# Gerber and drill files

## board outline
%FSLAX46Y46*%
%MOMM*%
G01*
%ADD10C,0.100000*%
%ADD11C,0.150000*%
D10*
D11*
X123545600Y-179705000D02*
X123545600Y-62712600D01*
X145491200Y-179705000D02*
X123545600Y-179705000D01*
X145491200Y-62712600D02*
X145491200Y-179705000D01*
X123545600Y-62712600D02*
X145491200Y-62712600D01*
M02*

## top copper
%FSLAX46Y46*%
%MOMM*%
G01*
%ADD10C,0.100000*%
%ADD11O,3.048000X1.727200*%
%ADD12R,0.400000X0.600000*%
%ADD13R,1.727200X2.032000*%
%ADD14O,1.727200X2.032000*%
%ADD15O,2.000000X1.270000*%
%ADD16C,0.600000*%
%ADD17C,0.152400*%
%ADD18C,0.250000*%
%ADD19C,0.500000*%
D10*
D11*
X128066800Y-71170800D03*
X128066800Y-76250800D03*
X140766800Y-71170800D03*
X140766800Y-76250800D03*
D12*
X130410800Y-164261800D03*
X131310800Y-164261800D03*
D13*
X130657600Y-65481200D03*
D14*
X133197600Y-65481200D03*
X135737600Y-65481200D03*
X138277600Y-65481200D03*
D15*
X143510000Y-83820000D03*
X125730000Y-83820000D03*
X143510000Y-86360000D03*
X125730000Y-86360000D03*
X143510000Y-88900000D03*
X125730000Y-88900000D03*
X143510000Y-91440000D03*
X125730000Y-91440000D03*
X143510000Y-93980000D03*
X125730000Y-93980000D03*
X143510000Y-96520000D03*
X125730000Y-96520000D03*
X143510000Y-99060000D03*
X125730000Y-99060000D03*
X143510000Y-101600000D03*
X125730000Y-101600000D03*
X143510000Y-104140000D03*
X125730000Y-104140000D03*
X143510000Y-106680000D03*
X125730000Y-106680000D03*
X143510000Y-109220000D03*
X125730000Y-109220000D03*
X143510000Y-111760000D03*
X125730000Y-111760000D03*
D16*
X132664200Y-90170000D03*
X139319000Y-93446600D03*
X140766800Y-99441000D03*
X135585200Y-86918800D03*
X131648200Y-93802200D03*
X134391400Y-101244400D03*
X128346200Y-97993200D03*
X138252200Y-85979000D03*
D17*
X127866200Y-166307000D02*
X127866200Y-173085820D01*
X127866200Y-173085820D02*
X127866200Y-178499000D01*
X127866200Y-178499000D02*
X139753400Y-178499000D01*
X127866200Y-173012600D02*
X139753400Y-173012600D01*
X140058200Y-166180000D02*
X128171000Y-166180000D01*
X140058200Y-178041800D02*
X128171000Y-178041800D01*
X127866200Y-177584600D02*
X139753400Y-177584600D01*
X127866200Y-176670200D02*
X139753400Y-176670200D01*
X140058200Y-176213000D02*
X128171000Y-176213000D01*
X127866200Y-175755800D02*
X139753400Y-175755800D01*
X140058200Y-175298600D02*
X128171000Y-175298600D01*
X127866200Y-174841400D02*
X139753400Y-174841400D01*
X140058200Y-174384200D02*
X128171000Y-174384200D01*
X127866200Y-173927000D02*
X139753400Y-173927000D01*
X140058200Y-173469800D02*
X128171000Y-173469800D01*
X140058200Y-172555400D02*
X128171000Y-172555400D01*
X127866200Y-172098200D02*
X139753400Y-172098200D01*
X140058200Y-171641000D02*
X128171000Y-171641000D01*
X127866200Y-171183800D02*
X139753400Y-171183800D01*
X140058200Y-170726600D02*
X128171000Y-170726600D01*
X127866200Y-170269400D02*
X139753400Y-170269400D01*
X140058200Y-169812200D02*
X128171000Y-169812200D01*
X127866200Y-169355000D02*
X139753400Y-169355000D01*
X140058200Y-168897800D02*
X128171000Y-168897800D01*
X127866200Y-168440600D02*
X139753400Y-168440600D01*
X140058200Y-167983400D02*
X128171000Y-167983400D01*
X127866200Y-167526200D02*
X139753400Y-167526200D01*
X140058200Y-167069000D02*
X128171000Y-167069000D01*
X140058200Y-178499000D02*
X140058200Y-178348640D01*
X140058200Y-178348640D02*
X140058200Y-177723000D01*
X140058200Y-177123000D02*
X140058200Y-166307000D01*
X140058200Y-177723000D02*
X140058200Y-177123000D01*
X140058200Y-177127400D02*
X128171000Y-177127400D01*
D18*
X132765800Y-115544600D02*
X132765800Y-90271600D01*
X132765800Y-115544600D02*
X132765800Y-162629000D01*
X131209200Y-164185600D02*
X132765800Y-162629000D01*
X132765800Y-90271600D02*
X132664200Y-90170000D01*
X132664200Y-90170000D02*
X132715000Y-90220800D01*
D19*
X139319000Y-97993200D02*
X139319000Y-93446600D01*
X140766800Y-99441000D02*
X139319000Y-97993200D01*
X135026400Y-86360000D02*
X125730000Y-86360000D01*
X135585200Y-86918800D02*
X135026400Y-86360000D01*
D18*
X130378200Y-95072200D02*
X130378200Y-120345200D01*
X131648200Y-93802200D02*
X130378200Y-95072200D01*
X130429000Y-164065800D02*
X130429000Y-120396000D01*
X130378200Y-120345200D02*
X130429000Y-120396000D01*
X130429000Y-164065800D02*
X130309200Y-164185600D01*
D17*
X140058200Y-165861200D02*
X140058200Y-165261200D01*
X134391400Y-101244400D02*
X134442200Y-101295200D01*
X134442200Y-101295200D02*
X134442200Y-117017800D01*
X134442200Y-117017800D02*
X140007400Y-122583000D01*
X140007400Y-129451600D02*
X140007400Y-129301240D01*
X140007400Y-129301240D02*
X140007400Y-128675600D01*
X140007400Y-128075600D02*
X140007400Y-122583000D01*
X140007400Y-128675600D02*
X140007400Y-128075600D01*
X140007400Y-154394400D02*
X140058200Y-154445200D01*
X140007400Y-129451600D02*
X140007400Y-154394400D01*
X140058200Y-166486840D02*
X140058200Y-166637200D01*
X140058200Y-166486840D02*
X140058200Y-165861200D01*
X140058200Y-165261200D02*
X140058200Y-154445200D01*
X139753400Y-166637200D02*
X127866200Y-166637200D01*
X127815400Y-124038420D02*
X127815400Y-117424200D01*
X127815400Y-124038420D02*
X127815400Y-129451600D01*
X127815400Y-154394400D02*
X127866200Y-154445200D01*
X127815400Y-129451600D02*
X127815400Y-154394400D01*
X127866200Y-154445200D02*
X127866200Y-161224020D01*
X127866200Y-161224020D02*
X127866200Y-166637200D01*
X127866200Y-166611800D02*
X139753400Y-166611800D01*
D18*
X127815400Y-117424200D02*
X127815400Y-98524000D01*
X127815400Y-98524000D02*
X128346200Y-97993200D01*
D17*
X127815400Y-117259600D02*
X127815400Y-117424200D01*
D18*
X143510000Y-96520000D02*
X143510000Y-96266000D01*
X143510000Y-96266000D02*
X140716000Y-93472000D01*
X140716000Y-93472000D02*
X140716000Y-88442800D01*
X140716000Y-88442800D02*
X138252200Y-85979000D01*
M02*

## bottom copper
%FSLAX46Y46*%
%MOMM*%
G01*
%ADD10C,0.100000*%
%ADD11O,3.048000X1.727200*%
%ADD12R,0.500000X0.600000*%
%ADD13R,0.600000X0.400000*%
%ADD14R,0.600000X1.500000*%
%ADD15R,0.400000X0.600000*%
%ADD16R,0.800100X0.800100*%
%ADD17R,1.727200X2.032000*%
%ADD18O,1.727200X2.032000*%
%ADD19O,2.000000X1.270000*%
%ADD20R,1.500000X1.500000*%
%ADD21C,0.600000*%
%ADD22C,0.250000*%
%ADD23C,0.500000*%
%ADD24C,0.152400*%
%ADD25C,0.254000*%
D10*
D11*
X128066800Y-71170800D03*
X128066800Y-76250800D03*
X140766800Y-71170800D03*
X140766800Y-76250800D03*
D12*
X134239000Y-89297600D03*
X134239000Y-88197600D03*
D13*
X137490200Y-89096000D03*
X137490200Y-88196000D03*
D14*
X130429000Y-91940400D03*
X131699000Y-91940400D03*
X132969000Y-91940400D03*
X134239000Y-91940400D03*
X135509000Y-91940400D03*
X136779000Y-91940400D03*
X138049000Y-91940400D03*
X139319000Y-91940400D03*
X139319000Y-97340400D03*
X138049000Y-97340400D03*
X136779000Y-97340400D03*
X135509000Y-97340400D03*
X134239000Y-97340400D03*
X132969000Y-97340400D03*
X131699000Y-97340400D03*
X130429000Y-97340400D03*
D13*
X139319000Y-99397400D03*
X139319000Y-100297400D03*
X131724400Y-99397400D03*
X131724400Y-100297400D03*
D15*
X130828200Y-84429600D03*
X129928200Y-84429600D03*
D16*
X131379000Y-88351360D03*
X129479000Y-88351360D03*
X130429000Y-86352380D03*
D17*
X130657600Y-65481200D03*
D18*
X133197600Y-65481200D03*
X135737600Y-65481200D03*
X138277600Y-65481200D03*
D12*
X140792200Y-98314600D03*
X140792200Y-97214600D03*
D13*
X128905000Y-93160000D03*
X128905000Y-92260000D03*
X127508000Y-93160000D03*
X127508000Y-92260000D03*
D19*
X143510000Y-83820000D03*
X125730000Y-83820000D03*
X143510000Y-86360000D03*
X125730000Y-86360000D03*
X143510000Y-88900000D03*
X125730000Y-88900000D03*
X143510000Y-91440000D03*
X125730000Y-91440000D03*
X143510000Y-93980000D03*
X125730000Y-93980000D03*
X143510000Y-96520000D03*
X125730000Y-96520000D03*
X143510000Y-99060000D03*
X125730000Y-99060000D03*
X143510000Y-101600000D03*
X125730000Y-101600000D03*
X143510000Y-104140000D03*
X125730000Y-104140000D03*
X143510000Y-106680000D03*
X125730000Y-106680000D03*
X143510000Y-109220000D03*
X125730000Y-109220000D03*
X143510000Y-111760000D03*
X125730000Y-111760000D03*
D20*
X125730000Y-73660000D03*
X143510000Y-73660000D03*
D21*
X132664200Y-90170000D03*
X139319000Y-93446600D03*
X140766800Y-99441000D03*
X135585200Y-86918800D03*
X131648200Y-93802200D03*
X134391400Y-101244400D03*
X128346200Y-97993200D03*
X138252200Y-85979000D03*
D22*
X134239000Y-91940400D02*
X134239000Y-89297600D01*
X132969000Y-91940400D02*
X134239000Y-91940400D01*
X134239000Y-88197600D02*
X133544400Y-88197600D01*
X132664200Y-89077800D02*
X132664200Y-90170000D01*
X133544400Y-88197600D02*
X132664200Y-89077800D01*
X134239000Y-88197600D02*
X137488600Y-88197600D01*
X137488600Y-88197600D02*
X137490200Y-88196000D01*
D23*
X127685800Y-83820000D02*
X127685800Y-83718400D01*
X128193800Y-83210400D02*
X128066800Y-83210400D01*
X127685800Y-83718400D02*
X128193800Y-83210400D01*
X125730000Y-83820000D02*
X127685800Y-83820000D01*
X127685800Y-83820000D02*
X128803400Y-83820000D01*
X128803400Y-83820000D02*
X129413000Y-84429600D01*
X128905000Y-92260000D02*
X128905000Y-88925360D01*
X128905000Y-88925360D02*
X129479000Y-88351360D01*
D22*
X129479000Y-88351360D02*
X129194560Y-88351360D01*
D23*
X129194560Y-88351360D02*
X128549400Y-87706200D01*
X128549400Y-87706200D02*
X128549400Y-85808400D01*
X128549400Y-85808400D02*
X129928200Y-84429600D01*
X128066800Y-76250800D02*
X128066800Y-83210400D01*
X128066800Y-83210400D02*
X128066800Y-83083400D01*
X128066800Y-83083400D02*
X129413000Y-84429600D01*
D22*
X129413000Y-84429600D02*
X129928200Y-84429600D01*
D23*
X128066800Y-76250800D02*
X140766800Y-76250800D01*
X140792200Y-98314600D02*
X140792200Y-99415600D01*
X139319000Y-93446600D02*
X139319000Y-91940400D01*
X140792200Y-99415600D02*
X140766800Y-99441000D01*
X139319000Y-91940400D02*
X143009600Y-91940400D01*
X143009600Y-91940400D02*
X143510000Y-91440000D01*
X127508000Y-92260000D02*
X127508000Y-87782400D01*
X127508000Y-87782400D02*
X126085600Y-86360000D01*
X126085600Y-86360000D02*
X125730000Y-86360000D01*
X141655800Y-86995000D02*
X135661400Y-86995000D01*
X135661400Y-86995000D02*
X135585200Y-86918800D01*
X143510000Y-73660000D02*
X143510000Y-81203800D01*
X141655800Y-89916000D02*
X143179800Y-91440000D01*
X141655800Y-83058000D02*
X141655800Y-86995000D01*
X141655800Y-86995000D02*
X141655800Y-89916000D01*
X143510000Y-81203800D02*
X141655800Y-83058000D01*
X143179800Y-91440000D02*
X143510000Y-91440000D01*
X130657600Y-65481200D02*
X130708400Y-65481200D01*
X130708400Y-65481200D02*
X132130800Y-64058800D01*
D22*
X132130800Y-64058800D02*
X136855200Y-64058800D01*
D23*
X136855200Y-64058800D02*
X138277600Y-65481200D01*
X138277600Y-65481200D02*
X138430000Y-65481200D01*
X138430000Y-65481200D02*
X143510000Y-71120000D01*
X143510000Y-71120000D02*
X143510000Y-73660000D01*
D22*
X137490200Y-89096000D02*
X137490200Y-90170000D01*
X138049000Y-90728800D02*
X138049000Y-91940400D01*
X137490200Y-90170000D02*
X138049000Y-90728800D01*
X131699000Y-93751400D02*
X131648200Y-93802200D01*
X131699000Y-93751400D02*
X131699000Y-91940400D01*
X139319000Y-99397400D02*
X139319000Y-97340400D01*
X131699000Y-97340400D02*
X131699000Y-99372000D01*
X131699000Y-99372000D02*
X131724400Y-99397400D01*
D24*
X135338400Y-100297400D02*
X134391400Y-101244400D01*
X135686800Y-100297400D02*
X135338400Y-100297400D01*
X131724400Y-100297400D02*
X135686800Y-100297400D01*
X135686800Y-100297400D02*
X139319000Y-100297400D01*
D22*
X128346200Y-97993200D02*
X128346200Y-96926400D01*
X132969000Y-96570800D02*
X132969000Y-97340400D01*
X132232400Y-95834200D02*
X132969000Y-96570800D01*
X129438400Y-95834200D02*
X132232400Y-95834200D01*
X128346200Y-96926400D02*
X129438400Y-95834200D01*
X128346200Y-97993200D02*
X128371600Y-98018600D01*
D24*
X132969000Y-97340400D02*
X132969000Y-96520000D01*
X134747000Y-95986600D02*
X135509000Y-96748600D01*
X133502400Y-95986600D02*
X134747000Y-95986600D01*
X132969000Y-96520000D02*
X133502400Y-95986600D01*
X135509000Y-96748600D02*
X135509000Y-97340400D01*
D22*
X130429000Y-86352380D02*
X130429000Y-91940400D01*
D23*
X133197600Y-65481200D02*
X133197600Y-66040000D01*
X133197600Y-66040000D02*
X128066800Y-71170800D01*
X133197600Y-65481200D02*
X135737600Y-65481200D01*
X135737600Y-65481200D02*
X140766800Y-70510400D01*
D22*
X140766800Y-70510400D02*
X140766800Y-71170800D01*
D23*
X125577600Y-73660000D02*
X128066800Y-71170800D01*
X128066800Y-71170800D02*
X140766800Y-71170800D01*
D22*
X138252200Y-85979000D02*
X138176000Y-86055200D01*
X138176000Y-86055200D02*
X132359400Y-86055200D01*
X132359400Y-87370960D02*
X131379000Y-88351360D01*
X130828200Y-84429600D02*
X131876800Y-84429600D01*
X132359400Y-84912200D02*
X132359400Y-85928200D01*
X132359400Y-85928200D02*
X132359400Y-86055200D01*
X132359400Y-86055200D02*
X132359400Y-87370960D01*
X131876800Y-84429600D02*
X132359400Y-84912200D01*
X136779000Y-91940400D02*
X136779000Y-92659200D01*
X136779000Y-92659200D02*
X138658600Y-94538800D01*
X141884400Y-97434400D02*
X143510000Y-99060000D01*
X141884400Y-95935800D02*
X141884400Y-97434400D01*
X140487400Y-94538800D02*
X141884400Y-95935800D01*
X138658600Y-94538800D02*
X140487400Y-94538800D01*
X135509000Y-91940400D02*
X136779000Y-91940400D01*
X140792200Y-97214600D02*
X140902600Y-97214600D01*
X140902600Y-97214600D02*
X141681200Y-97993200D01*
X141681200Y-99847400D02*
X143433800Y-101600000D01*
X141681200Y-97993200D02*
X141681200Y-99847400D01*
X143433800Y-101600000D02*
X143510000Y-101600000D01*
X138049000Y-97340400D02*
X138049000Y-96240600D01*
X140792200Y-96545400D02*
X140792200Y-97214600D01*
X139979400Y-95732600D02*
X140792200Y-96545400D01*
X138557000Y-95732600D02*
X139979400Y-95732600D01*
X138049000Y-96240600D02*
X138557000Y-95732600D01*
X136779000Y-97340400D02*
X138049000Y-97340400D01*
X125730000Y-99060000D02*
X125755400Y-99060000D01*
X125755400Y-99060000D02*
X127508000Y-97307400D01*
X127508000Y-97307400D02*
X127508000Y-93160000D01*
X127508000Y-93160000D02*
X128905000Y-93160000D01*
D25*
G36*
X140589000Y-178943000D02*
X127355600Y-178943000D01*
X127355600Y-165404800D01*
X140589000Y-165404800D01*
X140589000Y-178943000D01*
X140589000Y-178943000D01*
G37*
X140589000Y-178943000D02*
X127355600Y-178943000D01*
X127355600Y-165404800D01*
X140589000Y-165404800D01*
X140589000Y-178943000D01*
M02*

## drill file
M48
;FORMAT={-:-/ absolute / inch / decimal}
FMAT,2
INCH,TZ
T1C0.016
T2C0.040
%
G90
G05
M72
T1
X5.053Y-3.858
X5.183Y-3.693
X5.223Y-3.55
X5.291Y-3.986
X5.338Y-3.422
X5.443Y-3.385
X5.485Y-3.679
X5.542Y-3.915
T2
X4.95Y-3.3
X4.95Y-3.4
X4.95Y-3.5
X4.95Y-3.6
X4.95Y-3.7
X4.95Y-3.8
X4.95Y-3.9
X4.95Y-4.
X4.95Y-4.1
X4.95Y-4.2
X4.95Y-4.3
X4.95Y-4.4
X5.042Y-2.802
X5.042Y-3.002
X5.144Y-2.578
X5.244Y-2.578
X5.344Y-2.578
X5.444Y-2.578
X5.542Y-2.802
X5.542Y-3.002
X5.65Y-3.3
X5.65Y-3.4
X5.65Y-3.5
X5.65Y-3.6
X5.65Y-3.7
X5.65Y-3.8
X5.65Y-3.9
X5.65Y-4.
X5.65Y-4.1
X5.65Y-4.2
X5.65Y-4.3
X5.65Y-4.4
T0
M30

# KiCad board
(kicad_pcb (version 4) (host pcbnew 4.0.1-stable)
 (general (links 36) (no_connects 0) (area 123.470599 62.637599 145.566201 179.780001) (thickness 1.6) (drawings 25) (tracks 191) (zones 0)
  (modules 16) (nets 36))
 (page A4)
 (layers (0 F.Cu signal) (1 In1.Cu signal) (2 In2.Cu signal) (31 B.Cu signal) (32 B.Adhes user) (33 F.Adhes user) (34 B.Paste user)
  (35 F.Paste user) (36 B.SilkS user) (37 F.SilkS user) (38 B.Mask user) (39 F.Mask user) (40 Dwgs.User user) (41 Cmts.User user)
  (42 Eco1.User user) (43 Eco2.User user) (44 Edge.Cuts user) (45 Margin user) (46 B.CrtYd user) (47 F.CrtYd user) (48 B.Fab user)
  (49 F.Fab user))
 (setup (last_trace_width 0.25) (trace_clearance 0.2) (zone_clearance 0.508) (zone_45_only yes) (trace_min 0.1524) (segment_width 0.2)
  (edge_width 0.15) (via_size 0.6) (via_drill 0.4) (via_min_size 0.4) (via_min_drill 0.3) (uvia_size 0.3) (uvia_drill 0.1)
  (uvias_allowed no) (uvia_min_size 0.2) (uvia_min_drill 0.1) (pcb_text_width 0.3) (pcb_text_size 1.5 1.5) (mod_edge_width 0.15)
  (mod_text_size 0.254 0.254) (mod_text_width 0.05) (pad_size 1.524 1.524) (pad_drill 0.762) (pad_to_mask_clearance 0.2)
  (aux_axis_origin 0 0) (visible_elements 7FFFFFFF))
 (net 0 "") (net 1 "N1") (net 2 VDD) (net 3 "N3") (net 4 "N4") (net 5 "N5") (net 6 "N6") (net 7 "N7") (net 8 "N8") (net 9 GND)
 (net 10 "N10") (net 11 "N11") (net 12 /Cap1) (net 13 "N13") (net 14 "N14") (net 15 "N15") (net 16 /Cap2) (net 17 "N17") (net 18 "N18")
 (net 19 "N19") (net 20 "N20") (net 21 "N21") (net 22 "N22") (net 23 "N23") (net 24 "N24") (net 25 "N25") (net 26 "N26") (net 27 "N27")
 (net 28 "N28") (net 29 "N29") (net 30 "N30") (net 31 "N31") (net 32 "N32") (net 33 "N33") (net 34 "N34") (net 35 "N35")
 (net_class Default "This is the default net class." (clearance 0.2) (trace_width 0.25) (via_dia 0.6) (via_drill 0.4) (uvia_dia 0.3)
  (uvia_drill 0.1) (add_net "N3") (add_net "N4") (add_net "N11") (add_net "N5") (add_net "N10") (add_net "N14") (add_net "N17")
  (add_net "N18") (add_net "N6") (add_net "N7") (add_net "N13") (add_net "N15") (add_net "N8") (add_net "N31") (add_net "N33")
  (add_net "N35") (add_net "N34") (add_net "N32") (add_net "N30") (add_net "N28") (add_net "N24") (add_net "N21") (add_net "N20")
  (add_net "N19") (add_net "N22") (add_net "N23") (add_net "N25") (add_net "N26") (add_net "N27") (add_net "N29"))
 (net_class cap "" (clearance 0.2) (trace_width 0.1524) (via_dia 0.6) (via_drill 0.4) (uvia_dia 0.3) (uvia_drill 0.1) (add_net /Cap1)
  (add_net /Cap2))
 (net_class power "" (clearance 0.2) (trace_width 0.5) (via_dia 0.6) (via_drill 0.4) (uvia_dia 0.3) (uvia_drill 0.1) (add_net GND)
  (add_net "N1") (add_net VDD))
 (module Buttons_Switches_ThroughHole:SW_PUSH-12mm (layer B.Cu) (at 134.4168 73.7108 180)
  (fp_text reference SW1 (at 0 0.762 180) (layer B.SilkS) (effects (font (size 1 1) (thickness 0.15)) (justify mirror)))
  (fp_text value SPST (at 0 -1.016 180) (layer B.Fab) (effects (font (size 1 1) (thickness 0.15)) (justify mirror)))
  (pad 1 thru_hole oval (at 6.35 2.54 180) (size 3.048 1.7272) (drill 1.016) (layers *.Cu *.Mask B.SilkS) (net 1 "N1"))
  (pad 2 thru_hole oval (at 6.35 -2.54 180) (size 3.048 1.7272) (drill 1.016) (layers *.Cu *.Mask B.SilkS) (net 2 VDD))
  (pad 1 thru_hole oval (at -6.35 2.54 180) (size 3.048 1.7272) (drill 1.016) (layers *.Cu *.Mask B.SilkS) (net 1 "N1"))
  (pad 2 thru_hole oval (at -6.35 -2.54 180) (size 3.048 1.7272) (drill 1.016) (layers *.Cu *.Mask B.SilkS) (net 2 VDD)))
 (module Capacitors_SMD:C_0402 (layer B.Cu) (at 134.239 88.7476 90)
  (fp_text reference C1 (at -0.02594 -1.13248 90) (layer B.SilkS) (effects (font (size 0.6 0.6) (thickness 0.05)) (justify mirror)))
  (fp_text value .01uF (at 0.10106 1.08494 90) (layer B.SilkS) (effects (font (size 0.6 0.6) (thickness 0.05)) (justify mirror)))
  (pad 1 smd rect (at -0.55 0 90) (size 0.6 0.5) (layers B.Cu B.Paste B.Mask) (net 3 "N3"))
  (pad 2 smd rect (at 0.55 0 90) (size 0.6 0.5) (layers B.Cu B.Paste B.Mask) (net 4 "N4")))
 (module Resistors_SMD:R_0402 (layer B.Cu) (at 137.4902 88.646 90)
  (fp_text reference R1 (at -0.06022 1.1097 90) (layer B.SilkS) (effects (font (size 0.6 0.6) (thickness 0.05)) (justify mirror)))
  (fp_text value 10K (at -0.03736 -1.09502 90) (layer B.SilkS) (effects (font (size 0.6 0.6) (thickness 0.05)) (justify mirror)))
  (pad 1 smd rect (at -0.45 0 90) (size 0.4 0.6) (layers B.Cu B.Paste B.Mask) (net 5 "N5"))
  (pad 2 smd rect (at 0.45 0 90) (size 0.4 0.6) (layers B.Cu B.Paste B.Mask) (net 4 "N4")))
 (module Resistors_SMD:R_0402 (layer F.Cu) (at 130.8608 164.2618)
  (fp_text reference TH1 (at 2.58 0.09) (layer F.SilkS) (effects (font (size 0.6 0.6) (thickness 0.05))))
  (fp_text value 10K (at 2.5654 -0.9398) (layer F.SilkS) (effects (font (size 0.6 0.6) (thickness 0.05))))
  (pad 1 smd rect (at -0.45 0) (size 0.4 0.6) (layers F.Cu F.Paste F.Mask) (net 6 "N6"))
  (pad 2 smd rect (at 0.45 0) (size 0.4 0.6) (layers F.Cu F.Paste F.Mask) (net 4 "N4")))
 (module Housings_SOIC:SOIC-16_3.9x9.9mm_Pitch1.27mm (layer B.Cu) (at 134.874 94.6404 270)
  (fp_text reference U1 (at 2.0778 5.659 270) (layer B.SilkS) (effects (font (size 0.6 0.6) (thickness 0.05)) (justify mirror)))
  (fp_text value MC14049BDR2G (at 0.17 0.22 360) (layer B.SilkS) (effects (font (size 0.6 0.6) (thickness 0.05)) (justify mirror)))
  (pad 1 smd rect (at -2.7 4.445 270) (size 1.5 0.6) (layers B.Cu B.Paste B.Mask) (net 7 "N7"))
  (pad 2 smd rect (at -2.7 3.175 270) (size 1.5 0.6) (layers B.Cu B.Paste B.Mask) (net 6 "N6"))
  (pad 3 smd rect (at -2.7 1.905 270) (size 1.5 0.6) (layers B.Cu B.Paste B.Mask) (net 3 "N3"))
  (pad 4 smd rect (at -2.7 0.635 270) (size 1.5 0.6) (layers B.Cu B.Paste B.Mask) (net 3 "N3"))
  (pad 5 smd rect (at -2.7 -0.635 270) (size 1.5 0.6) (layers B.Cu B.Paste B.Mask) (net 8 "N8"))
  (pad 6 smd rect (at -2.7 -1.905 270) (size 1.5 0.6) (layers B.Cu B.Paste B.Mask) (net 8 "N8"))
  (pad 7 smd rect (at -2.7 -3.175 270) (size 1.5 0.6) (layers B.Cu B.Paste B.Mask) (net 5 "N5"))
  (pad 8 smd rect (at -2.7 -4.445 270) (size 1.5 0.6) (layers B.Cu B.Paste B.Mask) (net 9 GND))
  (pad 9 smd rect (at 2.7 -4.445 270) (size 1.5 0.6) (layers B.Cu B.Paste B.Mask) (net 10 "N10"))
  (pad 10 smd rect (at 2.7 -3.175 270) (size 1.5 0.6) (layers B.Cu B.Paste B.Mask) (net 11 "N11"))
  (pad 11 smd rect (at 2.7 -1.905 270) (size 1.5 0.6) (layers B.Cu B.Paste B.Mask) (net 11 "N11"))
  (pad 12 smd rect (at 2.7 -0.635 270) (size 1.5 0.6) (layers B.Cu B.Paste B.Mask) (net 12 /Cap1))
  (pad 13 smd rect (at 2.7 0.635 270) (size 1.5 0.6) (layers B.Cu B.Paste B.Mask) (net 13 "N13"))
  (pad 14 smd rect (at 2.7 1.905 270) (size 1.5 0.6) (layers B.Cu B.Paste B.Mask) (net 12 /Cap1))
  (pad 15 smd rect (at 2.7 3.175 270) (size 1.5 0.6) (layers B.Cu B.Paste B.Mask) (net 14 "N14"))
  (pad 16 smd rect (at 2.7 4.445 270) (size 1.5 0.6) (layers B.Cu B.Paste B.Mask) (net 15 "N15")))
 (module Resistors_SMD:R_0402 (layer B.Cu) (at 139.319 99.8474 270)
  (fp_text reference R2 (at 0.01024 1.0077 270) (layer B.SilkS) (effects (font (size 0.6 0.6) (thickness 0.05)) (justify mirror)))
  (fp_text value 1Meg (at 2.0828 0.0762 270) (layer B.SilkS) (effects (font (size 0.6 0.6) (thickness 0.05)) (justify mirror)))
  (pad 1 smd rect (at -0.45 0 270) (size 0.4 0.6) (layers B.Cu B.Paste B.Mask) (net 10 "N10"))
  (pad 2 smd rect (at 0.45 0 270) (size 0.4 0.6) (layers B.Cu B.Paste B.Mask) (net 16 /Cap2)))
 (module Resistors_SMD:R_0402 (layer B.Cu) (at 131.7244 99.8474 270)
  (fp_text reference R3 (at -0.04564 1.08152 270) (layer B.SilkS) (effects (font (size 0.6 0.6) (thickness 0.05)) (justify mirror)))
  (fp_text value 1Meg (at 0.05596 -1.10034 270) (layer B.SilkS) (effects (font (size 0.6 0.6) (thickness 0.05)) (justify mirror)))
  (pad 1 smd rect (at -0.45 0 270) (size 0.4 0.6) (layers B.Cu B.Paste B.Mask) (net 14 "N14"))
  (pad 2 smd rect (at 0.45 0 270) (size 0.4 0.6) (layers B.Cu B.Paste B.Mask) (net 16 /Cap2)))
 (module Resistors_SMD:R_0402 (layer B.Cu) (at 130.3782 84.4296 180)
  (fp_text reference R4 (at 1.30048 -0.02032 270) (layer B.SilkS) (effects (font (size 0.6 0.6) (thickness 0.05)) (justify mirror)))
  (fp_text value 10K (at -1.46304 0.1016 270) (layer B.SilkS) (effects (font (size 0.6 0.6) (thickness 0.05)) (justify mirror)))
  (pad 1 smd rect (at -0.45 0 180) (size 0.4 0.6) (layers B.Cu B.Paste B.Mask) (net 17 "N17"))
  (pad 2 smd rect (at 0.45 0 180) (size 0.4 0.6) (layers B.Cu B.Paste B.Mask) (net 2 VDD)))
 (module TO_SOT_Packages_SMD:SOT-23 (layer B.Cu) (at 130.429 87.3506 180)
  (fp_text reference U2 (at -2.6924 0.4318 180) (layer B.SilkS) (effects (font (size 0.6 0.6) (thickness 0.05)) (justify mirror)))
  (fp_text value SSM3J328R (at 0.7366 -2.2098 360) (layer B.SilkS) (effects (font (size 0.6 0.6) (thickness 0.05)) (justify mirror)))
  (pad 1 smd rect (at -0.95 -1.00076 180) (size 0.8001 0.8001) (layers B.Cu B.Paste B.Mask) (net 17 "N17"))
  (pad 2 smd rect (at 0.95 -1.00076 180) (size 0.8001 0.8001) (layers B.Cu B.Paste B.Mask) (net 2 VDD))
  (pad 3 smd rect (at 0 0.99822 180) (size 0.8001 0.8001) (layers B.Cu B.Paste B.Mask) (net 7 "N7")))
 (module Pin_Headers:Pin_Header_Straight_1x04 (layer F.Cu) (at 130.6576 65.4812 90)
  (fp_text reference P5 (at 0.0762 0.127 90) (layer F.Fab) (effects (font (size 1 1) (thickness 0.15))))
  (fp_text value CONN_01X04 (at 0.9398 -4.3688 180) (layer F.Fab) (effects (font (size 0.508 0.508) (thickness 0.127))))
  (pad 1 thru_hole rect (at 0 0 90) (size 2.032 1.7272) (drill 1.016) (layers *.Cu *.Mask F.SilkS) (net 9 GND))
  (pad 2 thru_hole oval (at 0 2.54 90) (size 2.032 1.7272) (drill 1.016) (layers *.Cu *.Mask F.SilkS) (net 1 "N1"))
  (pad 3 thru_hole oval (at 0 5.08 90) (size 2.032 1.7272) (drill 1.016) (layers *.Cu *.Mask F.SilkS) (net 1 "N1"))
  (pad 4 thru_hole oval (at 0 7.62 90) (size 2.032 1.7272) (drill 1.016) (layers *.Cu *.Mask F.SilkS) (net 9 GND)))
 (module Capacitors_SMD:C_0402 (layer B.Cu) (at 140.7922 97.7646 90)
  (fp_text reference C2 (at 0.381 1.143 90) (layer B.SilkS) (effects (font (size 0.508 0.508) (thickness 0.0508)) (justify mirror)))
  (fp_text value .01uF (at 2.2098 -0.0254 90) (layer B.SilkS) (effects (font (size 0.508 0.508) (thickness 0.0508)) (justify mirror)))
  (pad 1 smd rect (at -0.55 0 90) (size 0.6 0.5) (layers B.Cu B.Paste B.Mask) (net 9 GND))
  (pad 2 smd rect (at 0.55 0 90) (size 0.6 0.5) (layers B.Cu B.Paste B.Mask) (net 11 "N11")))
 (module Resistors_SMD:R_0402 (layer B.Cu) (at 128.905 92.71 90)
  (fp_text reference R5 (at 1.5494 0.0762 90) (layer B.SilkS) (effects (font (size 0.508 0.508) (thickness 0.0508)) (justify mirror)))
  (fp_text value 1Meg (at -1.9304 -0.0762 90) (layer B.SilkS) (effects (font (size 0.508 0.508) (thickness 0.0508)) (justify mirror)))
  (pad 1 smd rect (at -0.45 0 90) (size 0.4 0.6) (layers B.Cu B.Paste B.Mask) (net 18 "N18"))
  (pad 2 smd rect (at 0.45 0 90) (size 0.4 0.6) (layers B.Cu B.Paste B.Mask) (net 2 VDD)))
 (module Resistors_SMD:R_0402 (layer B.Cu) (at 127.508 92.71 90)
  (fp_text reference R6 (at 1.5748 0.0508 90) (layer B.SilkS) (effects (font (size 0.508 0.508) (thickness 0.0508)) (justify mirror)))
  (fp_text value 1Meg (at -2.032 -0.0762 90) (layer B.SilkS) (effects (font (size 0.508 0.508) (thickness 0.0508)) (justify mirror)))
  (pad 1 smd rect (at -0.45 0 90) (size 0.4 0.6) (layers B.Cu B.Paste B.Mask) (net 18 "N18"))
  (pad 2 smd rect (at 0.45 0 90) (size 0.4 0.6) (layers B.Cu B.Paste B.Mask) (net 9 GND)))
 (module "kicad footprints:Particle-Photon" (layer F.Cu) (at 134.62 97.79 270)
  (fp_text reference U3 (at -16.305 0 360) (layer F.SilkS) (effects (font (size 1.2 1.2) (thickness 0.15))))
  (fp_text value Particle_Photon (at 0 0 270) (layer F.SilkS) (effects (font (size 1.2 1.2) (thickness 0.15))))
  (pad 24 thru_hole oval (at -13.97 -8.89 270) (size 1.27 2) (drill 1.016) (layers *.Cu *.Mask F.SilkS) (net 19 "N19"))
  (pad 1 thru_hole oval (at -13.97 8.89 270) (size 1.27 2) (drill 1.016) (layers *.Cu *.Mask F.SilkS) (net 2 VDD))
  (pad 23 thru_hole oval (at -11.43 -8.89 270) (size 1.27 2) (drill 1.016) (layers *.Cu *.Mask F.SilkS) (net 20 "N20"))
  (pad 2 thru_hole oval (at -11.43 8.89 270) (size 1.27 2) (drill 1.016) (layers *.Cu *.Mask F.SilkS) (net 9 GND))
  (pad 22 thru_hole oval (at -8.89 -8.89 270) (size 1.27 2) (drill 1.016) (layers *.Cu *.Mask F.SilkS) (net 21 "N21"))
  (pad 3 thru_hole oval (at -8.89 8.89 270) (size 1.27 2) (drill 1.016) (layers *.Cu *.Mask F.SilkS) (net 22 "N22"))
  (pad 21 thru_hole oval (at -6.35 -8.89 270) (size 1.27 2) (drill 1.016) (layers *.Cu *.Mask F.SilkS) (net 9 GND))
  (pad 4 thru_hole oval (at -6.35 8.89 270) (size 1.27 2) (drill 1.016) (layers *.Cu *.Mask F.SilkS) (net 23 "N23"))
  (pad 20 thru_hole oval (at -3.81 -8.89 270) (size 1.27 2) (drill 1.016) (layers *.Cu *.Mask F.SilkS) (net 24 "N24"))
  (pad 5 thru_hole oval (at -3.81 8.89 270) (size 1.27 2) (drill 1.016) (layers *.Cu *.Mask F.SilkS) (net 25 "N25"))
  (pad 19 thru_hole oval (at -1.27 -8.89 270) (size 1.27 2) (drill 1.016) (layers *.Cu *.Mask F.SilkS) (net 17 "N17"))
  (pad 6 thru_hole oval (at -1.27 8.89 270) (size 1.27 2) (drill 1.016) (layers *.Cu *.Mask F.SilkS) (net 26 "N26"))
  (pad 18 thru_hole oval (at 1.27 -8.89 270) (size 1.27 2) (drill 1.016) (layers *.Cu *.Mask F.SilkS) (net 8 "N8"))
  (pad 7 thru_hole oval (at 1.27 8.89 270) (size 1.27 2) (drill 1.016) (layers *.Cu *.Mask F.SilkS) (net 18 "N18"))
  (pad 17 thru_hole oval (at 3.81 -8.89 270) (size 1.27 2) (drill 1.016) (layers *.Cu *.Mask F.SilkS) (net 11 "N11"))
  (pad 8 thru_hole oval (at 3.81 8.89 270) (size 1.27 2) (drill 1.016) (layers *.Cu *.Mask F.SilkS) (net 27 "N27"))
  (pad 16 thru_hole oval (at 6.35 -8.89 270) (size 1.27 2) (drill 1.016) (layers *.Cu *.Mask F.SilkS) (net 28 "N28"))
  (pad 9 thru_hole oval (at 6.35 8.89 270) (size 1.27 2) (drill 1.016) (layers *.Cu *.Mask F.SilkS) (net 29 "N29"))
  (pad 15 thru_hole oval (at 8.89 -8.89 270) (size 1.27 2) (drill 1.016) (layers *.Cu *.Mask F.SilkS) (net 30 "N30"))
  (pad 10 thru_hole oval (at 8.89 8.89 270) (size 1.27 2) (drill 1.016) (layers *.Cu *.Mask F.SilkS) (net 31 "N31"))
  (pad 14 thru_hole oval (at 11.43 -8.89 270) (size 1.27 2) (drill 1.016) (layers *.Cu *.Mask F.SilkS) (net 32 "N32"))
  (pad 11 thru_hole oval (at 11.43 8.89 270) (size 1.27 2) (drill 1.016) (layers *.Cu *.Mask F.SilkS) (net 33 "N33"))
  (pad 13 thru_hole oval (at 13.97 -8.89 270) (size 1.27 2) (drill 1.016) (layers *.Cu *.Mask F.SilkS) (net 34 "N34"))
  (pad 12 thru_hole oval (at 13.97 8.89 270) (size 1.27 2) (drill 1.016) (layers *.Cu *.Mask F.SilkS) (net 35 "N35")))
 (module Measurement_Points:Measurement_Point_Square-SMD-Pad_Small (layer B.Cu) (at 125.73 73.66)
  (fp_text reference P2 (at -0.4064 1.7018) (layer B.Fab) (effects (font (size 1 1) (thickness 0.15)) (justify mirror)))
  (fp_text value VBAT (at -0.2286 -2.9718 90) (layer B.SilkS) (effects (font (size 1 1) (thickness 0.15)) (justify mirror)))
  (pad 1 smd rect (at 0 0) (size 1.5 1.5) (layers B.Cu B.Mask) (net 1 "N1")))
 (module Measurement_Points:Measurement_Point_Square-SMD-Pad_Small (layer B.Cu) (at 143.51 73.66)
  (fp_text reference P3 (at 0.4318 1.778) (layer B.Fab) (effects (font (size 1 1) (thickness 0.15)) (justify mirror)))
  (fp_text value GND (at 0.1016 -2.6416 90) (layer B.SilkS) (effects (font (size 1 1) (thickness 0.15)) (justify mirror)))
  (pad 1 smd rect (at 0 0) (size 1.5 1.5) (layers B.Cu B.Mask) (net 9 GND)))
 (gr_line (start 123.5456 179.705) (end 123.5456 62.7126) (angle 90) (layer Edge.Cuts) (width 0.15))
 (gr_line (start 145.4912 179.705) (end 123.5456 179.705) (angle 90) (layer Edge.Cuts) (width 0.15))
 (gr_line (start 145.4912 62.7126) (end 145.4912 179.705) (angle 90) (layer Edge.Cuts) (width 0.15))
 (gr_line (start 123.5456 62.7126) (end 145.4912 62.7126) (angle 90) (layer Edge.Cuts) (width 0.15))
 (segment (start 127.8662 166.307) (end 127.8662 173.08582) (width 0.1524) (layer F.Cu) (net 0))
 (segment (start 127.8662 173.08582) (end 127.8662 178.499) (width 0.1524) (layer F.Cu) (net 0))
 (segment (start 127.8662 178.499) (end 139.7534 178.499) (width 0.1524) (layer F.Cu) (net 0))
 (segment (start 127.8662 173.0126) (end 139.7534 173.0126) (width 0.1524) (layer F.Cu) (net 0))
 (segment (start 140.0582 166.18) (end 128.171 166.18) (width 0.1524) (layer F.Cu) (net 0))
 (segment (start 140.0582 178.0418) (end 128.171 178.0418) (width 0.1524) (layer F.Cu) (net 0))
 (segment (start 127.8662 177.5846) (end 139.7534 177.5846) (width 0.1524) (layer F.Cu) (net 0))
 (segment (start 127.8662 176.6702) (end 139.7534 176.6702) (width 0.1524) (layer F.Cu) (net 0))
 (segment (start 140.0582 176.213) (end 128.171 176.213) (width 0.1524) (layer F.Cu) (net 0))
 (segment (start 127.8662 175.7558) (end 139.7534 175.7558) (width 0.1524) (layer F.Cu) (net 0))
 (segment (start 140.0582 175.2986) (end 128.171 175.2986) (width 0.1524) (layer F.Cu) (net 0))
 (segment (start 127.8662 174.8414) (end 139.7534 174.8414) (width 0.1524) (layer F.Cu) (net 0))
 (segment (start 140.0582 174.3842) (end 128.171 174.3842) (width 0.1524) (layer F.Cu) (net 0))
 (segment (start 127.8662 173.927) (end 139.7534 173.927) (width 0.1524) (layer F.Cu) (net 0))
 (segment (start 140.0582 173.4698) (end 128.171 173.4698) (width 0.1524) (layer F.Cu) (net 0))
 (segment (start 140.0582 172.5554) (end 128.171 172.5554) (width 0.1524) (layer F.Cu) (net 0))
 (segment (start 127.8662 172.0982) (end 139.7534 172.0982) (width 0.1524) (layer F.Cu) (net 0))
 (segment (start 140.0582 171.641) (end 128.171 171.641) (width 0.1524) (layer F.Cu) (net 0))
 (segment (start 127.8662 171.1838) (end 139.7534 171.1838) (width 0.1524) (layer F.Cu) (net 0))
 (segment (start 140.0582 170.7266) (end 128.171 170.7266) (width 0.1524) (layer F.Cu) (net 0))
 (segment (start 127.8662 170.2694) (end 139.7534 170.2694) (width 0.1524) (layer F.Cu) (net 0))
 (segment (start 140.0582 169.8122) (end 128.171 169.8122) (width 0.1524) (layer F.Cu) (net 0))
 (segment (start 127.8662 169.355) (end 139.7534 169.355) (width 0.1524) (layer F.Cu) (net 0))
 (segment (start 140.0582 168.8978) (end 128.171 168.8978) (width 0.1524) (layer F.Cu) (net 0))
 (segment (start 127.8662 168.4406) (end 139.7534 168.4406) (width 0.1524) (layer F.Cu) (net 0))
 (segment (start 140.0582 167.9834) (end 128.171 167.9834) (width 0.1524) (layer F.Cu) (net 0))
 (segment (start 127.8662 167.5262) (end 139.7534 167.5262) (width 0.1524) (layer F.Cu) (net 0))
 (segment (start 140.0582 167.069) (end 128.171 167.069) (width 0.1524) (layer F.Cu) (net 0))
 (segment (start 140.0582 178.499) (end 140.0582 178.34864) (width 0.1524) (layer F.Cu) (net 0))
 (segment (start 140.0582 178.34864) (end 140.0582 177.723) (width 0.1524) (layer F.Cu) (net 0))
 (segment (start 140.0582 177.123) (end 140.0582 166.307) (width 0.1524) (layer F.Cu) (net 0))
 (segment (start 140.0582 177.723) (end 140.0582 177.123) (width 0.1524) (layer F.Cu) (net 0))
 (segment (start 140.0582 177.1274) (end 128.171 177.1274) (width 0.1524) (layer F.Cu) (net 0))
 (segment (start 134.239 91.9404) (end 134.239 89.2976) (width 0.25) (layer B.Cu) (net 3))
 (segment (start 132.969 91.9404) (end 134.239 91.9404) (width 0.25) (layer B.Cu) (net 3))
 (segment (start 132.7658 115.5446) (end 132.7658 90.2716) (width 0.25) (layer F.Cu) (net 4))
 (segment (start 132.7658 115.5446) (end 132.7658 162.629) (width 0.25) (layer F.Cu) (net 4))
 (segment (start 131.2092 164.1856) (end 132.7658 162.629) (width 0.25) (layer F.Cu) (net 4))
 (segment (start 132.7658 90.2716) (end 132.6642 90.17) (width 0.25) (layer F.Cu) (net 4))
 (segment (start 134.239 88.1976) (end 133.5444 88.1976) (width 0.25) (layer B.Cu) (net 4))
 (segment (start 132.6642 90.17) (end 132.715 90.2208) (width 0.25) (layer F.Cu) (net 4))
 (via (at 132.6642 90.17) (size 0.6) (drill 0.4) (layers F.Cu B.Cu) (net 4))
 (segment (start 132.6642 89.0778) (end 132.6642 90.17) (width 0.25) (layer B.Cu) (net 4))
 (segment (start 133.5444 88.1976) (end 132.6642 89.0778) (width 0.25) (layer B.Cu) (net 4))
 (segment (start 134.239 88.1976) (end 137.4886 88.1976) (width 0.25) (layer B.Cu) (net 4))
 (segment (start 137.4886 88.1976) (end 137.4902 88.196) (width 0.25) (layer B.Cu) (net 4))
 (segment (start 127.6858 83.82) (end 127.6858 83.7184) (width 0.5) (layer B.Cu) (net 2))
 (segment (start 128.1938 83.2104) (end 128.0668 83.2104) (width 0.5) (layer B.Cu) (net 2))
 (segment (start 127.6858 83.7184) (end 128.1938 83.2104) (width 0.5) (layer B.Cu) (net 2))
 (segment (start 125.73 83.82) (end 127.6858 83.82) (width 0.5) (layer B.Cu) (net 2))
 (segment (start 127.6858 83.82) (end 128.8034 83.82) (width 0.5) (layer B.Cu) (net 2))
 (segment (start 128.8034 83.82) (end 129.413 84.4296) (width 0.5) (layer B.Cu) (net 2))
 (segment (start 128.905 92.26) (end 128.905 88.92536) (width 0.5) (layer B.Cu) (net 2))
 (segment (start 128.905 88.92536) (end 129.479 88.35136) (width 0.5) (layer B.Cu) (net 2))
 (segment (start 129.479 88.35136) (end 129.19456 88.35136) (width 0.25) (layer B.Cu) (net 2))
 (segment (start 129.19456 88.35136) (end 128.5494 87.7062) (width 0.5) (layer B.Cu) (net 2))
 (segment (start 128.5494 87.7062) (end 128.5494 85.8084) (width 0.5) (layer B.Cu) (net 2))
 (segment (start 128.5494 85.8084) (end 129.9282 84.4296) (width 0.5) (layer B.Cu) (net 2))
 (segment (start 128.0668 76.2508) (end 128.0668 83.2104) (width 0.5) (layer B.Cu) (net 2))
 (segment (start 128.0668 83.2104) (end 128.0668 83.0834) (width 0.5) (layer B.Cu) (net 2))
 (segment (start 128.0668 83.0834) (end 129.413 84.4296) (width 0.5) (layer B.Cu) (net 2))
 (segment (start 129.413 84.4296) (end 129.9282 84.4296) (width 0.25) (layer B.Cu) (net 2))
 (segment (start 128.0668 76.2508) (end 140.7668 76.2508) (width 0.5) (layer B.Cu) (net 2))
 (segment (start 140.7922 98.3146) (end 140.7922 99.4156) (width 0.5) (layer B.Cu) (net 9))
 (segment (start 139.319 93.4466) (end 139.319 91.9404) (width 0.5) (layer B.Cu) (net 9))
 (via (at 139.319 93.4466) (size 0.6) (drill 0.4) (layers F.Cu B.Cu) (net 9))
 (segment (start 139.319 97.9932) (end 139.319 93.4466) (width 0.5) (layer F.Cu) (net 9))
 (segment (start 140.7668 99.441) (end 139.319 97.9932) (width 0.5) (layer F.Cu) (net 9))
 (via (at 140.7668 99.441) (size 0.6) (drill 0.4) (layers F.Cu B.Cu) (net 9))
 (segment (start 140.7922 99.4156) (end 140.7668 99.441) (width 0.5) (layer B.Cu) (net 9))
 (segment (start 139.319 91.9404) (end 143.0096 91.9404) (width 0.5) (layer B.Cu) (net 9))
 (segment (start 143.0096 91.9404) (end 143.51 91.44) (width 0.5) (layer B.Cu) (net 9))
 (segment (start 127.508 92.26) (end 127.508 87.7824) (width 0.5) (layer B.Cu) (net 9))
 (segment (start 127.508 87.7824) (end 126.0856 86.36) (width 0.5) (layer B.Cu) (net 9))
 (segment (start 126.0856 86.36) (end 125.73 86.36) (width 0.5) (layer B.Cu) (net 9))
 (segment (start 141.6558 86.995) (end 135.6614 86.995) (width 0.5) (layer B.Cu) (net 9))
 (segment (start 135.0264 86.36) (end 125.73 86.36) (width 0.5) (layer F.Cu) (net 9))
 (segment (start 135.5852 86.9188) (end 135.0264 86.36) (width 0.5) (layer F.Cu) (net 9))
 (via (at 135.5852 86.9188) (size 0.6) (drill 0.4) (layers F.Cu B.Cu) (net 9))
 (segment (start 135.6614 86.995) (end 135.5852 86.9188) (width 0.5) (layer B.Cu) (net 9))
 (segment (start 143.51 73.66) (end 143.51 81.2038) (width 0.5) (layer B.Cu) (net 9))
 (segment (start 141.6558 89.916) (end 143.1798 91.44) (width 0.5) (layer B.Cu) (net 9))
 (segment (start 141.6558 83.058) (end 141.6558 86.995) (width 0.5) (layer B.Cu) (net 9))
 (segment (start 141.6558 86.995) (end 141.6558 89.916) (width 0.5) (layer B.Cu) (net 9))
 (segment (start 143.51 81.2038) (end 141.6558 83.058) (width 0.5) (layer B.Cu) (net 9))
 (segment (start 143.1798 91.44) (end 143.51 91.44) (width 0.5) (layer B.Cu) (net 9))
 (segment (start 130.6576 65.4812) (end 130.7084 65.4812) (width 0.5) (layer B.Cu) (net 9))
 (segment (start 130.7084 65.4812) (end 132.1308 64.0588) (width 0.5) (layer B.Cu) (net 9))
 (segment (start 132.1308 64.0588) (end 136.8552 64.0588) (width 0.25) (layer B.Cu) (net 9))
 (segment (start 136.8552 64.0588) (end 138.2776 65.4812) (width 0.5) (layer B.Cu) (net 9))
 (segment (start 138.2776 65.4812) (end 138.43 65.4812) (width 0.5) (layer B.Cu) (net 9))
 (segment (start 138.43 65.4812) (end 143.51 71.12) (width 0.5) (layer B.Cu) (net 9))
 (segment (start 143.51 71.12) (end 143.51 73.66) (width 0.5) (layer B.Cu) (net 9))
 (segment (start 137.4902 89.096) (end 137.4902 90.17) (width 0.25) (layer B.Cu) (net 5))
 (segment (start 138.049 90.7288) (end 138.049 91.9404) (width 0.25) (layer B.Cu) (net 5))
 (segment (start 137.4902 90.17) (end 138.049 90.7288) (width 0.25) (layer B.Cu) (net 5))
 (segment (start 130.3782 95.0722) (end 130.3782 120.3452) (width 0.25) (layer F.Cu) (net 6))
 (segment (start 131.699 93.7514) (end 131.6482 93.8022) (width 0.25) (layer B.Cu) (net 6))
 (via (at 131.6482 93.8022) (size 0.6) (drill 0.4) (layers F.Cu B.Cu) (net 6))
 (segment (start 131.6482 93.8022) (end 130.3782 95.0722) (width 0.25) (layer F.Cu) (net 6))
 (segment (start 130.429 164.0658) (end 130.429 120.396) (width 0.25) (layer F.Cu) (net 6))
 (segment (start 131.699 93.7514) (end 131.699 91.9404) (width 0.25) (layer B.Cu) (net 6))
 (segment (start 130.3782 120.3452) (end 130.429 120.396) (width 0.25) (layer F.Cu) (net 6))
 (segment (start 130.429 164.0658) (end 130.3092 164.1856) (width 0.25) (layer F.Cu) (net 6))
 (segment (start 139.319 99.3974) (end 139.319 97.3404) (width 0.25) (layer B.Cu) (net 10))
 (segment (start 131.699 97.3404) (end 131.699 99.372) (width 0.25) (layer B.Cu) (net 14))
 (segment (start 131.699 99.372) (end 131.7244 99.3974) (width 0.25) (layer B.Cu) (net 14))
 (segment (start 140.0582 165.8612) (end 140.0582 165.2612) (width 0.1524) (layer F.Cu) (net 16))
 (segment (start 135.3384 100.2974) (end 134.3914 101.2444) (width 0.1524) (layer B.Cu) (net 16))
 (via (at 134.3914 101.2444) (size 0.6) (drill 0.4) (layers F.Cu B.Cu) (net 16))
 (segment (start 134.3914 101.2444) (end 134.4422 101.2952) (width 0.1524) (layer F.Cu) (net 16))
 (segment (start 134.4422 101.2952) (end 134.4422 117.0178) (width 0.1524) (layer F.Cu) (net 16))
 (segment (start 134.4422 117.0178) (end 140.0074 122.583) (width 0.1524) (layer F.Cu) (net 16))
 (segment (start 135.6868 100.2974) (end 135.3384 100.2974) (width 0.1524) (layer B.Cu) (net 16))
 (segment (start 140.0074 129.4516) (end 140.0074 129.30124) (width 0.1524) (layer F.Cu) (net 16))
 (segment (start 140.0074 129.30124) (end 140.0074 128.6756) (width 0.1524) (layer F.Cu) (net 16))
 (segment (start 140.0074 128.0756) (end 140.0074 122.583) (width 0.1524) (layer F.Cu) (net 16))
 (segment (start 140.0074 128.6756) (end 140.0074 128.0756) (width 0.1524) (layer F.Cu) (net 16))
 (segment (start 140.0074 154.3944) (end 140.0582 154.4452) (width 0.1524) (layer F.Cu) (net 16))
 (segment (start 140.0074 129.4516) (end 140.0074 154.3944) (width 0.1524) (layer F.Cu) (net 16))
 (segment (start 140.0582 166.48684) (end 140.0582 166.6372) (width 0.1524) (layer F.Cu) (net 16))
 (segment (start 140.0582 166.48684) (end 140.0582 165.8612) (width 0.1524) (layer F.Cu) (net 16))
 (segment (start 140.0582 165.2612) (end 140.0582 154.4452) (width 0.1524) (layer F.Cu) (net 16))
 (segment (start 131.7244 100.2974) (end 135.6868 100.2974) (width 0.1524) (layer B.Cu) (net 16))
 (segment (start 135.6868 100.2974) (end 139.319 100.2974) (width 0.1524) (layer B.Cu) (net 16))
 (segment (start 139.7534 166.6372) (end 127.8662 166.6372) (width 0.1524) (layer F.Cu) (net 12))
 (segment (start 127.8154 124.03842) (end 127.8154 117.4242) (width 0.1524) (layer F.Cu) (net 12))
 (segment (start 127.8154 124.03842) (end 127.8154 129.4516) (width 0.1524) (layer F.Cu) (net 12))
 (segment (start 127.8154 154.3944) (end 127.8662 154.4452) (width 0.1524) (layer F.Cu) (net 12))
 (segment (start 127.8154 129.4516) (end 127.8154 154.3944) (width 0.1524) (layer F.Cu) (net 12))
 (segment (start 127.8662 154.4452) (end 127.8662 161.22402) (width 0.1524) (layer F.Cu) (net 12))
 (segment (start 127.8662 161.22402) (end 127.8662 166.6372) (width 0.1524) (layer F.Cu) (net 12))
 (segment (start 127.8662 166.6118) (end 139.7534 166.6118) (width 0.1524) (layer F.Cu) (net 12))
 (segment (start 128.3462 97.9932) (end 128.3462 96.9264) (width 0.25) (layer B.Cu) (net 12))
 (segment (start 132.969 96.5708) (end 132.969 97.3404) (width 0.25) (layer B.Cu) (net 12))
 (segment (start 132.2324 95.8342) (end 132.969 96.5708) (width 0.25) (layer B.Cu) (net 12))
 (segment (start 129.4384 95.8342) (end 132.2324 95.8342) (width 0.25) (layer B.Cu) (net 12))
 (segment (start 128.3462 96.9264) (end 129.4384 95.8342) (width 0.25) (layer B.Cu) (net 12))
 (segment (start 127.8154 117.4242) (end 127.8154 98.524) (width 0.25) (layer F.Cu) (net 12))
 (segment (start 128.3462 97.9932) (end 128.3716 98.0186) (width 0.25) (layer B.Cu) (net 12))
 (via (at 128.3462 97.9932) (size 0.6) (drill 0.4) (layers F.Cu B.Cu) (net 12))
 (segment (start 127.8154 98.524) (end 128.3462 97.9932) (width 0.25) (layer F.Cu) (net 12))
 (segment (start 127.8154 117.2596) (end 127.8154 117.4242) (width 0.1524) (layer F.Cu) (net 12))
 (segment (start 132.969 97.3404) (end 132.969 96.52) (width 0.1524) (layer B.Cu) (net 12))
 (segment (start 134.747 95.9866) (end 135.509 96.7486) (width 0.1524) (layer B.Cu) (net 12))
 (segment (start 133.5024 95.9866) (end 134.747 95.9866) (width 0.1524) (layer B.Cu) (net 12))
 (segment (start 132.969 96.52) (end 133.5024 95.9866) (width 0.1524) (layer B.Cu) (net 12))
 (segment (start 135.509 96.7486) (end 135.509 97.3404) (width 0.1524) (layer B.Cu) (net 12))
 (segment (start 130.429 86.35238) (end 130.429 91.9404) (width 0.25) (layer B.Cu) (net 7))
 (segment (start 133.1976 65.4812) (end 133.1976 66.04) (width 0.5) (layer B.Cu) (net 1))
 (segment (start 133.1976 66.04) (end 128.0668 71.1708) (width 0.5) (layer B.Cu) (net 1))
 (segment (start 133.1976 65.4812) (end 135.7376 65.4812) (width 0.5) (layer B.Cu) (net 1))
 (segment (start 135.7376 65.4812) (end 140.7668 70.5104) (width 0.5) (layer B.Cu) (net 1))
 (segment (start 140.7668 70.5104) (end 140.7668 71.1708) (width 0.25) (layer B.Cu) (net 1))
 (segment (start 125.5776 73.66) (end 128.0668 71.1708) (width 0.5) (layer B.Cu) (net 1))
 (segment (start 128.0668 71.1708) (end 140.7668 71.1708) (width 0.5) (layer B.Cu) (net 1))
 (segment (start 143.51 96.52) (end 143.51 96.266) (width 0.25) (layer F.Cu) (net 17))
 (segment (start 143.51 96.266) (end 140.716 93.472) (width 0.25) (layer F.Cu) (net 17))
 (segment (start 140.716 93.472) (end 140.716 88.4428) (width 0.25) (layer F.Cu) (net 17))
 (segment (start 140.716 88.4428) (end 138.2522 85.979) (width 0.25) (layer F.Cu) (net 17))
 (via (at 138.2522 85.979) (size 0.6) (drill 0.4) (layers F.Cu B.Cu) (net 17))
 (segment (start 138.2522 85.979) (end 138.176 86.0552) (width 0.25) (layer B.Cu) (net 17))
 (segment (start 138.176 86.0552) (end 132.3594 86.0552) (width 0.25) (layer B.Cu) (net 17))
 (segment (start 132.3594 87.37096) (end 131.379 88.35136) (width 0.25) (layer B.Cu) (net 17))
 (segment (start 130.8282 84.4296) (end 131.8768 84.4296) (width 0.25) (layer B.Cu) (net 17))
 (segment (start 132.3594 84.9122) (end 132.3594 85.9282) (width 0.25) (layer B.Cu) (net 17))
 (segment (start 132.3594 85.9282) (end 132.3594 86.0552) (width 0.25) (layer B.Cu) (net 17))
 (segment (start 132.3594 86.0552) (end 132.3594 87.37096) (width 0.25) (layer B.Cu) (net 17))
 (segment (start 131.8768 84.4296) (end 132.3594 84.9122) (width 0.25) (layer B.Cu) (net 17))
 (segment (start 136.779 91.9404) (end 136.779 92.6592) (width 0.25) (layer B.Cu) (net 8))
 (segment (start 136.779 92.6592) (end 138.6586 94.5388) (width 0.25) (layer B.Cu) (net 8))
 (segment (start 141.8844 97.4344) (end 143.51 99.06) (width 0.25) (layer B.Cu) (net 8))
 (segment (start 141.8844 95.9358) (end 141.8844 97.4344) (width 0.25) (layer B.Cu) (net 8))
 (segment (start 140.4874 94.5388) (end 141.8844 95.9358) (width 0.25) (layer B.Cu) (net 8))
 (segment (start 138.6586 94.5388) (end 140.4874 94.5388) (width 0.25) (layer B.Cu) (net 8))
 (segment (start 135.509 91.9404) (end 136.779 91.9404) (width 0.25) (layer B.Cu) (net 8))
 (segment (start 140.7922 97.2146) (end 140.9026 97.2146) (width 0.25) (layer B.Cu) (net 11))
 (segment (start 140.9026 97.2146) (end 141.6812 97.9932) (width 0.25) (layer B.Cu) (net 11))
 (segment (start 141.6812 99.8474) (end 143.4338 101.6) (width 0.25) (layer B.Cu) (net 11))
 (segment (start 141.6812 97.9932) (end 141.6812 99.8474) (width 0.25) (layer B.Cu) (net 11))
 (segment (start 143.4338 101.6) (end 143.51 101.6) (width 0.25) (layer B.Cu) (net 11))
 (segment (start 138.049 97.3404) (end 138.049 96.2406) (width 0.25) (layer B.Cu) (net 11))
 (segment (start 140.7922 96.5454) (end 140.7922 97.2146) (width 0.25) (layer B.Cu) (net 11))
 (segment (start 139.9794 95.7326) (end 140.7922 96.5454) (width 0.25) (layer B.Cu) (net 11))
 (segment (start 138.557 95.7326) (end 139.9794 95.7326) (width 0.25) (layer B.Cu) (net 11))
 (segment (start 138.049 96.2406) (end 138.557 95.7326) (width 0.25) (layer B.Cu) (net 11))
 (segment (start 136.779 97.3404) (end 138.049 97.3404) (width 0.25) (layer B.Cu) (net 11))
 (segment (start 125.73 99.06) (end 125.7554 99.06) (width 0.25) (layer B.Cu) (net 18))
 (segment (start 125.7554 99.06) (end 127.508 97.3074) (width 0.25) (layer B.Cu) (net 18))
 (segment (start 127.508 97.3074) (end 127.508 93.16) (width 0.25) (layer B.Cu) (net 18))
 (segment (start 127.508 93.16) (end 128.905 93.16) (width 0.25) (layer B.Cu) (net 18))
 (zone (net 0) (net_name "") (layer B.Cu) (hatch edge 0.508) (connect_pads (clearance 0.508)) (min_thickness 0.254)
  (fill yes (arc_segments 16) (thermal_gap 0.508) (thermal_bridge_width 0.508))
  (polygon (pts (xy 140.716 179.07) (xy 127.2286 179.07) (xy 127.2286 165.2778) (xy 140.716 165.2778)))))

